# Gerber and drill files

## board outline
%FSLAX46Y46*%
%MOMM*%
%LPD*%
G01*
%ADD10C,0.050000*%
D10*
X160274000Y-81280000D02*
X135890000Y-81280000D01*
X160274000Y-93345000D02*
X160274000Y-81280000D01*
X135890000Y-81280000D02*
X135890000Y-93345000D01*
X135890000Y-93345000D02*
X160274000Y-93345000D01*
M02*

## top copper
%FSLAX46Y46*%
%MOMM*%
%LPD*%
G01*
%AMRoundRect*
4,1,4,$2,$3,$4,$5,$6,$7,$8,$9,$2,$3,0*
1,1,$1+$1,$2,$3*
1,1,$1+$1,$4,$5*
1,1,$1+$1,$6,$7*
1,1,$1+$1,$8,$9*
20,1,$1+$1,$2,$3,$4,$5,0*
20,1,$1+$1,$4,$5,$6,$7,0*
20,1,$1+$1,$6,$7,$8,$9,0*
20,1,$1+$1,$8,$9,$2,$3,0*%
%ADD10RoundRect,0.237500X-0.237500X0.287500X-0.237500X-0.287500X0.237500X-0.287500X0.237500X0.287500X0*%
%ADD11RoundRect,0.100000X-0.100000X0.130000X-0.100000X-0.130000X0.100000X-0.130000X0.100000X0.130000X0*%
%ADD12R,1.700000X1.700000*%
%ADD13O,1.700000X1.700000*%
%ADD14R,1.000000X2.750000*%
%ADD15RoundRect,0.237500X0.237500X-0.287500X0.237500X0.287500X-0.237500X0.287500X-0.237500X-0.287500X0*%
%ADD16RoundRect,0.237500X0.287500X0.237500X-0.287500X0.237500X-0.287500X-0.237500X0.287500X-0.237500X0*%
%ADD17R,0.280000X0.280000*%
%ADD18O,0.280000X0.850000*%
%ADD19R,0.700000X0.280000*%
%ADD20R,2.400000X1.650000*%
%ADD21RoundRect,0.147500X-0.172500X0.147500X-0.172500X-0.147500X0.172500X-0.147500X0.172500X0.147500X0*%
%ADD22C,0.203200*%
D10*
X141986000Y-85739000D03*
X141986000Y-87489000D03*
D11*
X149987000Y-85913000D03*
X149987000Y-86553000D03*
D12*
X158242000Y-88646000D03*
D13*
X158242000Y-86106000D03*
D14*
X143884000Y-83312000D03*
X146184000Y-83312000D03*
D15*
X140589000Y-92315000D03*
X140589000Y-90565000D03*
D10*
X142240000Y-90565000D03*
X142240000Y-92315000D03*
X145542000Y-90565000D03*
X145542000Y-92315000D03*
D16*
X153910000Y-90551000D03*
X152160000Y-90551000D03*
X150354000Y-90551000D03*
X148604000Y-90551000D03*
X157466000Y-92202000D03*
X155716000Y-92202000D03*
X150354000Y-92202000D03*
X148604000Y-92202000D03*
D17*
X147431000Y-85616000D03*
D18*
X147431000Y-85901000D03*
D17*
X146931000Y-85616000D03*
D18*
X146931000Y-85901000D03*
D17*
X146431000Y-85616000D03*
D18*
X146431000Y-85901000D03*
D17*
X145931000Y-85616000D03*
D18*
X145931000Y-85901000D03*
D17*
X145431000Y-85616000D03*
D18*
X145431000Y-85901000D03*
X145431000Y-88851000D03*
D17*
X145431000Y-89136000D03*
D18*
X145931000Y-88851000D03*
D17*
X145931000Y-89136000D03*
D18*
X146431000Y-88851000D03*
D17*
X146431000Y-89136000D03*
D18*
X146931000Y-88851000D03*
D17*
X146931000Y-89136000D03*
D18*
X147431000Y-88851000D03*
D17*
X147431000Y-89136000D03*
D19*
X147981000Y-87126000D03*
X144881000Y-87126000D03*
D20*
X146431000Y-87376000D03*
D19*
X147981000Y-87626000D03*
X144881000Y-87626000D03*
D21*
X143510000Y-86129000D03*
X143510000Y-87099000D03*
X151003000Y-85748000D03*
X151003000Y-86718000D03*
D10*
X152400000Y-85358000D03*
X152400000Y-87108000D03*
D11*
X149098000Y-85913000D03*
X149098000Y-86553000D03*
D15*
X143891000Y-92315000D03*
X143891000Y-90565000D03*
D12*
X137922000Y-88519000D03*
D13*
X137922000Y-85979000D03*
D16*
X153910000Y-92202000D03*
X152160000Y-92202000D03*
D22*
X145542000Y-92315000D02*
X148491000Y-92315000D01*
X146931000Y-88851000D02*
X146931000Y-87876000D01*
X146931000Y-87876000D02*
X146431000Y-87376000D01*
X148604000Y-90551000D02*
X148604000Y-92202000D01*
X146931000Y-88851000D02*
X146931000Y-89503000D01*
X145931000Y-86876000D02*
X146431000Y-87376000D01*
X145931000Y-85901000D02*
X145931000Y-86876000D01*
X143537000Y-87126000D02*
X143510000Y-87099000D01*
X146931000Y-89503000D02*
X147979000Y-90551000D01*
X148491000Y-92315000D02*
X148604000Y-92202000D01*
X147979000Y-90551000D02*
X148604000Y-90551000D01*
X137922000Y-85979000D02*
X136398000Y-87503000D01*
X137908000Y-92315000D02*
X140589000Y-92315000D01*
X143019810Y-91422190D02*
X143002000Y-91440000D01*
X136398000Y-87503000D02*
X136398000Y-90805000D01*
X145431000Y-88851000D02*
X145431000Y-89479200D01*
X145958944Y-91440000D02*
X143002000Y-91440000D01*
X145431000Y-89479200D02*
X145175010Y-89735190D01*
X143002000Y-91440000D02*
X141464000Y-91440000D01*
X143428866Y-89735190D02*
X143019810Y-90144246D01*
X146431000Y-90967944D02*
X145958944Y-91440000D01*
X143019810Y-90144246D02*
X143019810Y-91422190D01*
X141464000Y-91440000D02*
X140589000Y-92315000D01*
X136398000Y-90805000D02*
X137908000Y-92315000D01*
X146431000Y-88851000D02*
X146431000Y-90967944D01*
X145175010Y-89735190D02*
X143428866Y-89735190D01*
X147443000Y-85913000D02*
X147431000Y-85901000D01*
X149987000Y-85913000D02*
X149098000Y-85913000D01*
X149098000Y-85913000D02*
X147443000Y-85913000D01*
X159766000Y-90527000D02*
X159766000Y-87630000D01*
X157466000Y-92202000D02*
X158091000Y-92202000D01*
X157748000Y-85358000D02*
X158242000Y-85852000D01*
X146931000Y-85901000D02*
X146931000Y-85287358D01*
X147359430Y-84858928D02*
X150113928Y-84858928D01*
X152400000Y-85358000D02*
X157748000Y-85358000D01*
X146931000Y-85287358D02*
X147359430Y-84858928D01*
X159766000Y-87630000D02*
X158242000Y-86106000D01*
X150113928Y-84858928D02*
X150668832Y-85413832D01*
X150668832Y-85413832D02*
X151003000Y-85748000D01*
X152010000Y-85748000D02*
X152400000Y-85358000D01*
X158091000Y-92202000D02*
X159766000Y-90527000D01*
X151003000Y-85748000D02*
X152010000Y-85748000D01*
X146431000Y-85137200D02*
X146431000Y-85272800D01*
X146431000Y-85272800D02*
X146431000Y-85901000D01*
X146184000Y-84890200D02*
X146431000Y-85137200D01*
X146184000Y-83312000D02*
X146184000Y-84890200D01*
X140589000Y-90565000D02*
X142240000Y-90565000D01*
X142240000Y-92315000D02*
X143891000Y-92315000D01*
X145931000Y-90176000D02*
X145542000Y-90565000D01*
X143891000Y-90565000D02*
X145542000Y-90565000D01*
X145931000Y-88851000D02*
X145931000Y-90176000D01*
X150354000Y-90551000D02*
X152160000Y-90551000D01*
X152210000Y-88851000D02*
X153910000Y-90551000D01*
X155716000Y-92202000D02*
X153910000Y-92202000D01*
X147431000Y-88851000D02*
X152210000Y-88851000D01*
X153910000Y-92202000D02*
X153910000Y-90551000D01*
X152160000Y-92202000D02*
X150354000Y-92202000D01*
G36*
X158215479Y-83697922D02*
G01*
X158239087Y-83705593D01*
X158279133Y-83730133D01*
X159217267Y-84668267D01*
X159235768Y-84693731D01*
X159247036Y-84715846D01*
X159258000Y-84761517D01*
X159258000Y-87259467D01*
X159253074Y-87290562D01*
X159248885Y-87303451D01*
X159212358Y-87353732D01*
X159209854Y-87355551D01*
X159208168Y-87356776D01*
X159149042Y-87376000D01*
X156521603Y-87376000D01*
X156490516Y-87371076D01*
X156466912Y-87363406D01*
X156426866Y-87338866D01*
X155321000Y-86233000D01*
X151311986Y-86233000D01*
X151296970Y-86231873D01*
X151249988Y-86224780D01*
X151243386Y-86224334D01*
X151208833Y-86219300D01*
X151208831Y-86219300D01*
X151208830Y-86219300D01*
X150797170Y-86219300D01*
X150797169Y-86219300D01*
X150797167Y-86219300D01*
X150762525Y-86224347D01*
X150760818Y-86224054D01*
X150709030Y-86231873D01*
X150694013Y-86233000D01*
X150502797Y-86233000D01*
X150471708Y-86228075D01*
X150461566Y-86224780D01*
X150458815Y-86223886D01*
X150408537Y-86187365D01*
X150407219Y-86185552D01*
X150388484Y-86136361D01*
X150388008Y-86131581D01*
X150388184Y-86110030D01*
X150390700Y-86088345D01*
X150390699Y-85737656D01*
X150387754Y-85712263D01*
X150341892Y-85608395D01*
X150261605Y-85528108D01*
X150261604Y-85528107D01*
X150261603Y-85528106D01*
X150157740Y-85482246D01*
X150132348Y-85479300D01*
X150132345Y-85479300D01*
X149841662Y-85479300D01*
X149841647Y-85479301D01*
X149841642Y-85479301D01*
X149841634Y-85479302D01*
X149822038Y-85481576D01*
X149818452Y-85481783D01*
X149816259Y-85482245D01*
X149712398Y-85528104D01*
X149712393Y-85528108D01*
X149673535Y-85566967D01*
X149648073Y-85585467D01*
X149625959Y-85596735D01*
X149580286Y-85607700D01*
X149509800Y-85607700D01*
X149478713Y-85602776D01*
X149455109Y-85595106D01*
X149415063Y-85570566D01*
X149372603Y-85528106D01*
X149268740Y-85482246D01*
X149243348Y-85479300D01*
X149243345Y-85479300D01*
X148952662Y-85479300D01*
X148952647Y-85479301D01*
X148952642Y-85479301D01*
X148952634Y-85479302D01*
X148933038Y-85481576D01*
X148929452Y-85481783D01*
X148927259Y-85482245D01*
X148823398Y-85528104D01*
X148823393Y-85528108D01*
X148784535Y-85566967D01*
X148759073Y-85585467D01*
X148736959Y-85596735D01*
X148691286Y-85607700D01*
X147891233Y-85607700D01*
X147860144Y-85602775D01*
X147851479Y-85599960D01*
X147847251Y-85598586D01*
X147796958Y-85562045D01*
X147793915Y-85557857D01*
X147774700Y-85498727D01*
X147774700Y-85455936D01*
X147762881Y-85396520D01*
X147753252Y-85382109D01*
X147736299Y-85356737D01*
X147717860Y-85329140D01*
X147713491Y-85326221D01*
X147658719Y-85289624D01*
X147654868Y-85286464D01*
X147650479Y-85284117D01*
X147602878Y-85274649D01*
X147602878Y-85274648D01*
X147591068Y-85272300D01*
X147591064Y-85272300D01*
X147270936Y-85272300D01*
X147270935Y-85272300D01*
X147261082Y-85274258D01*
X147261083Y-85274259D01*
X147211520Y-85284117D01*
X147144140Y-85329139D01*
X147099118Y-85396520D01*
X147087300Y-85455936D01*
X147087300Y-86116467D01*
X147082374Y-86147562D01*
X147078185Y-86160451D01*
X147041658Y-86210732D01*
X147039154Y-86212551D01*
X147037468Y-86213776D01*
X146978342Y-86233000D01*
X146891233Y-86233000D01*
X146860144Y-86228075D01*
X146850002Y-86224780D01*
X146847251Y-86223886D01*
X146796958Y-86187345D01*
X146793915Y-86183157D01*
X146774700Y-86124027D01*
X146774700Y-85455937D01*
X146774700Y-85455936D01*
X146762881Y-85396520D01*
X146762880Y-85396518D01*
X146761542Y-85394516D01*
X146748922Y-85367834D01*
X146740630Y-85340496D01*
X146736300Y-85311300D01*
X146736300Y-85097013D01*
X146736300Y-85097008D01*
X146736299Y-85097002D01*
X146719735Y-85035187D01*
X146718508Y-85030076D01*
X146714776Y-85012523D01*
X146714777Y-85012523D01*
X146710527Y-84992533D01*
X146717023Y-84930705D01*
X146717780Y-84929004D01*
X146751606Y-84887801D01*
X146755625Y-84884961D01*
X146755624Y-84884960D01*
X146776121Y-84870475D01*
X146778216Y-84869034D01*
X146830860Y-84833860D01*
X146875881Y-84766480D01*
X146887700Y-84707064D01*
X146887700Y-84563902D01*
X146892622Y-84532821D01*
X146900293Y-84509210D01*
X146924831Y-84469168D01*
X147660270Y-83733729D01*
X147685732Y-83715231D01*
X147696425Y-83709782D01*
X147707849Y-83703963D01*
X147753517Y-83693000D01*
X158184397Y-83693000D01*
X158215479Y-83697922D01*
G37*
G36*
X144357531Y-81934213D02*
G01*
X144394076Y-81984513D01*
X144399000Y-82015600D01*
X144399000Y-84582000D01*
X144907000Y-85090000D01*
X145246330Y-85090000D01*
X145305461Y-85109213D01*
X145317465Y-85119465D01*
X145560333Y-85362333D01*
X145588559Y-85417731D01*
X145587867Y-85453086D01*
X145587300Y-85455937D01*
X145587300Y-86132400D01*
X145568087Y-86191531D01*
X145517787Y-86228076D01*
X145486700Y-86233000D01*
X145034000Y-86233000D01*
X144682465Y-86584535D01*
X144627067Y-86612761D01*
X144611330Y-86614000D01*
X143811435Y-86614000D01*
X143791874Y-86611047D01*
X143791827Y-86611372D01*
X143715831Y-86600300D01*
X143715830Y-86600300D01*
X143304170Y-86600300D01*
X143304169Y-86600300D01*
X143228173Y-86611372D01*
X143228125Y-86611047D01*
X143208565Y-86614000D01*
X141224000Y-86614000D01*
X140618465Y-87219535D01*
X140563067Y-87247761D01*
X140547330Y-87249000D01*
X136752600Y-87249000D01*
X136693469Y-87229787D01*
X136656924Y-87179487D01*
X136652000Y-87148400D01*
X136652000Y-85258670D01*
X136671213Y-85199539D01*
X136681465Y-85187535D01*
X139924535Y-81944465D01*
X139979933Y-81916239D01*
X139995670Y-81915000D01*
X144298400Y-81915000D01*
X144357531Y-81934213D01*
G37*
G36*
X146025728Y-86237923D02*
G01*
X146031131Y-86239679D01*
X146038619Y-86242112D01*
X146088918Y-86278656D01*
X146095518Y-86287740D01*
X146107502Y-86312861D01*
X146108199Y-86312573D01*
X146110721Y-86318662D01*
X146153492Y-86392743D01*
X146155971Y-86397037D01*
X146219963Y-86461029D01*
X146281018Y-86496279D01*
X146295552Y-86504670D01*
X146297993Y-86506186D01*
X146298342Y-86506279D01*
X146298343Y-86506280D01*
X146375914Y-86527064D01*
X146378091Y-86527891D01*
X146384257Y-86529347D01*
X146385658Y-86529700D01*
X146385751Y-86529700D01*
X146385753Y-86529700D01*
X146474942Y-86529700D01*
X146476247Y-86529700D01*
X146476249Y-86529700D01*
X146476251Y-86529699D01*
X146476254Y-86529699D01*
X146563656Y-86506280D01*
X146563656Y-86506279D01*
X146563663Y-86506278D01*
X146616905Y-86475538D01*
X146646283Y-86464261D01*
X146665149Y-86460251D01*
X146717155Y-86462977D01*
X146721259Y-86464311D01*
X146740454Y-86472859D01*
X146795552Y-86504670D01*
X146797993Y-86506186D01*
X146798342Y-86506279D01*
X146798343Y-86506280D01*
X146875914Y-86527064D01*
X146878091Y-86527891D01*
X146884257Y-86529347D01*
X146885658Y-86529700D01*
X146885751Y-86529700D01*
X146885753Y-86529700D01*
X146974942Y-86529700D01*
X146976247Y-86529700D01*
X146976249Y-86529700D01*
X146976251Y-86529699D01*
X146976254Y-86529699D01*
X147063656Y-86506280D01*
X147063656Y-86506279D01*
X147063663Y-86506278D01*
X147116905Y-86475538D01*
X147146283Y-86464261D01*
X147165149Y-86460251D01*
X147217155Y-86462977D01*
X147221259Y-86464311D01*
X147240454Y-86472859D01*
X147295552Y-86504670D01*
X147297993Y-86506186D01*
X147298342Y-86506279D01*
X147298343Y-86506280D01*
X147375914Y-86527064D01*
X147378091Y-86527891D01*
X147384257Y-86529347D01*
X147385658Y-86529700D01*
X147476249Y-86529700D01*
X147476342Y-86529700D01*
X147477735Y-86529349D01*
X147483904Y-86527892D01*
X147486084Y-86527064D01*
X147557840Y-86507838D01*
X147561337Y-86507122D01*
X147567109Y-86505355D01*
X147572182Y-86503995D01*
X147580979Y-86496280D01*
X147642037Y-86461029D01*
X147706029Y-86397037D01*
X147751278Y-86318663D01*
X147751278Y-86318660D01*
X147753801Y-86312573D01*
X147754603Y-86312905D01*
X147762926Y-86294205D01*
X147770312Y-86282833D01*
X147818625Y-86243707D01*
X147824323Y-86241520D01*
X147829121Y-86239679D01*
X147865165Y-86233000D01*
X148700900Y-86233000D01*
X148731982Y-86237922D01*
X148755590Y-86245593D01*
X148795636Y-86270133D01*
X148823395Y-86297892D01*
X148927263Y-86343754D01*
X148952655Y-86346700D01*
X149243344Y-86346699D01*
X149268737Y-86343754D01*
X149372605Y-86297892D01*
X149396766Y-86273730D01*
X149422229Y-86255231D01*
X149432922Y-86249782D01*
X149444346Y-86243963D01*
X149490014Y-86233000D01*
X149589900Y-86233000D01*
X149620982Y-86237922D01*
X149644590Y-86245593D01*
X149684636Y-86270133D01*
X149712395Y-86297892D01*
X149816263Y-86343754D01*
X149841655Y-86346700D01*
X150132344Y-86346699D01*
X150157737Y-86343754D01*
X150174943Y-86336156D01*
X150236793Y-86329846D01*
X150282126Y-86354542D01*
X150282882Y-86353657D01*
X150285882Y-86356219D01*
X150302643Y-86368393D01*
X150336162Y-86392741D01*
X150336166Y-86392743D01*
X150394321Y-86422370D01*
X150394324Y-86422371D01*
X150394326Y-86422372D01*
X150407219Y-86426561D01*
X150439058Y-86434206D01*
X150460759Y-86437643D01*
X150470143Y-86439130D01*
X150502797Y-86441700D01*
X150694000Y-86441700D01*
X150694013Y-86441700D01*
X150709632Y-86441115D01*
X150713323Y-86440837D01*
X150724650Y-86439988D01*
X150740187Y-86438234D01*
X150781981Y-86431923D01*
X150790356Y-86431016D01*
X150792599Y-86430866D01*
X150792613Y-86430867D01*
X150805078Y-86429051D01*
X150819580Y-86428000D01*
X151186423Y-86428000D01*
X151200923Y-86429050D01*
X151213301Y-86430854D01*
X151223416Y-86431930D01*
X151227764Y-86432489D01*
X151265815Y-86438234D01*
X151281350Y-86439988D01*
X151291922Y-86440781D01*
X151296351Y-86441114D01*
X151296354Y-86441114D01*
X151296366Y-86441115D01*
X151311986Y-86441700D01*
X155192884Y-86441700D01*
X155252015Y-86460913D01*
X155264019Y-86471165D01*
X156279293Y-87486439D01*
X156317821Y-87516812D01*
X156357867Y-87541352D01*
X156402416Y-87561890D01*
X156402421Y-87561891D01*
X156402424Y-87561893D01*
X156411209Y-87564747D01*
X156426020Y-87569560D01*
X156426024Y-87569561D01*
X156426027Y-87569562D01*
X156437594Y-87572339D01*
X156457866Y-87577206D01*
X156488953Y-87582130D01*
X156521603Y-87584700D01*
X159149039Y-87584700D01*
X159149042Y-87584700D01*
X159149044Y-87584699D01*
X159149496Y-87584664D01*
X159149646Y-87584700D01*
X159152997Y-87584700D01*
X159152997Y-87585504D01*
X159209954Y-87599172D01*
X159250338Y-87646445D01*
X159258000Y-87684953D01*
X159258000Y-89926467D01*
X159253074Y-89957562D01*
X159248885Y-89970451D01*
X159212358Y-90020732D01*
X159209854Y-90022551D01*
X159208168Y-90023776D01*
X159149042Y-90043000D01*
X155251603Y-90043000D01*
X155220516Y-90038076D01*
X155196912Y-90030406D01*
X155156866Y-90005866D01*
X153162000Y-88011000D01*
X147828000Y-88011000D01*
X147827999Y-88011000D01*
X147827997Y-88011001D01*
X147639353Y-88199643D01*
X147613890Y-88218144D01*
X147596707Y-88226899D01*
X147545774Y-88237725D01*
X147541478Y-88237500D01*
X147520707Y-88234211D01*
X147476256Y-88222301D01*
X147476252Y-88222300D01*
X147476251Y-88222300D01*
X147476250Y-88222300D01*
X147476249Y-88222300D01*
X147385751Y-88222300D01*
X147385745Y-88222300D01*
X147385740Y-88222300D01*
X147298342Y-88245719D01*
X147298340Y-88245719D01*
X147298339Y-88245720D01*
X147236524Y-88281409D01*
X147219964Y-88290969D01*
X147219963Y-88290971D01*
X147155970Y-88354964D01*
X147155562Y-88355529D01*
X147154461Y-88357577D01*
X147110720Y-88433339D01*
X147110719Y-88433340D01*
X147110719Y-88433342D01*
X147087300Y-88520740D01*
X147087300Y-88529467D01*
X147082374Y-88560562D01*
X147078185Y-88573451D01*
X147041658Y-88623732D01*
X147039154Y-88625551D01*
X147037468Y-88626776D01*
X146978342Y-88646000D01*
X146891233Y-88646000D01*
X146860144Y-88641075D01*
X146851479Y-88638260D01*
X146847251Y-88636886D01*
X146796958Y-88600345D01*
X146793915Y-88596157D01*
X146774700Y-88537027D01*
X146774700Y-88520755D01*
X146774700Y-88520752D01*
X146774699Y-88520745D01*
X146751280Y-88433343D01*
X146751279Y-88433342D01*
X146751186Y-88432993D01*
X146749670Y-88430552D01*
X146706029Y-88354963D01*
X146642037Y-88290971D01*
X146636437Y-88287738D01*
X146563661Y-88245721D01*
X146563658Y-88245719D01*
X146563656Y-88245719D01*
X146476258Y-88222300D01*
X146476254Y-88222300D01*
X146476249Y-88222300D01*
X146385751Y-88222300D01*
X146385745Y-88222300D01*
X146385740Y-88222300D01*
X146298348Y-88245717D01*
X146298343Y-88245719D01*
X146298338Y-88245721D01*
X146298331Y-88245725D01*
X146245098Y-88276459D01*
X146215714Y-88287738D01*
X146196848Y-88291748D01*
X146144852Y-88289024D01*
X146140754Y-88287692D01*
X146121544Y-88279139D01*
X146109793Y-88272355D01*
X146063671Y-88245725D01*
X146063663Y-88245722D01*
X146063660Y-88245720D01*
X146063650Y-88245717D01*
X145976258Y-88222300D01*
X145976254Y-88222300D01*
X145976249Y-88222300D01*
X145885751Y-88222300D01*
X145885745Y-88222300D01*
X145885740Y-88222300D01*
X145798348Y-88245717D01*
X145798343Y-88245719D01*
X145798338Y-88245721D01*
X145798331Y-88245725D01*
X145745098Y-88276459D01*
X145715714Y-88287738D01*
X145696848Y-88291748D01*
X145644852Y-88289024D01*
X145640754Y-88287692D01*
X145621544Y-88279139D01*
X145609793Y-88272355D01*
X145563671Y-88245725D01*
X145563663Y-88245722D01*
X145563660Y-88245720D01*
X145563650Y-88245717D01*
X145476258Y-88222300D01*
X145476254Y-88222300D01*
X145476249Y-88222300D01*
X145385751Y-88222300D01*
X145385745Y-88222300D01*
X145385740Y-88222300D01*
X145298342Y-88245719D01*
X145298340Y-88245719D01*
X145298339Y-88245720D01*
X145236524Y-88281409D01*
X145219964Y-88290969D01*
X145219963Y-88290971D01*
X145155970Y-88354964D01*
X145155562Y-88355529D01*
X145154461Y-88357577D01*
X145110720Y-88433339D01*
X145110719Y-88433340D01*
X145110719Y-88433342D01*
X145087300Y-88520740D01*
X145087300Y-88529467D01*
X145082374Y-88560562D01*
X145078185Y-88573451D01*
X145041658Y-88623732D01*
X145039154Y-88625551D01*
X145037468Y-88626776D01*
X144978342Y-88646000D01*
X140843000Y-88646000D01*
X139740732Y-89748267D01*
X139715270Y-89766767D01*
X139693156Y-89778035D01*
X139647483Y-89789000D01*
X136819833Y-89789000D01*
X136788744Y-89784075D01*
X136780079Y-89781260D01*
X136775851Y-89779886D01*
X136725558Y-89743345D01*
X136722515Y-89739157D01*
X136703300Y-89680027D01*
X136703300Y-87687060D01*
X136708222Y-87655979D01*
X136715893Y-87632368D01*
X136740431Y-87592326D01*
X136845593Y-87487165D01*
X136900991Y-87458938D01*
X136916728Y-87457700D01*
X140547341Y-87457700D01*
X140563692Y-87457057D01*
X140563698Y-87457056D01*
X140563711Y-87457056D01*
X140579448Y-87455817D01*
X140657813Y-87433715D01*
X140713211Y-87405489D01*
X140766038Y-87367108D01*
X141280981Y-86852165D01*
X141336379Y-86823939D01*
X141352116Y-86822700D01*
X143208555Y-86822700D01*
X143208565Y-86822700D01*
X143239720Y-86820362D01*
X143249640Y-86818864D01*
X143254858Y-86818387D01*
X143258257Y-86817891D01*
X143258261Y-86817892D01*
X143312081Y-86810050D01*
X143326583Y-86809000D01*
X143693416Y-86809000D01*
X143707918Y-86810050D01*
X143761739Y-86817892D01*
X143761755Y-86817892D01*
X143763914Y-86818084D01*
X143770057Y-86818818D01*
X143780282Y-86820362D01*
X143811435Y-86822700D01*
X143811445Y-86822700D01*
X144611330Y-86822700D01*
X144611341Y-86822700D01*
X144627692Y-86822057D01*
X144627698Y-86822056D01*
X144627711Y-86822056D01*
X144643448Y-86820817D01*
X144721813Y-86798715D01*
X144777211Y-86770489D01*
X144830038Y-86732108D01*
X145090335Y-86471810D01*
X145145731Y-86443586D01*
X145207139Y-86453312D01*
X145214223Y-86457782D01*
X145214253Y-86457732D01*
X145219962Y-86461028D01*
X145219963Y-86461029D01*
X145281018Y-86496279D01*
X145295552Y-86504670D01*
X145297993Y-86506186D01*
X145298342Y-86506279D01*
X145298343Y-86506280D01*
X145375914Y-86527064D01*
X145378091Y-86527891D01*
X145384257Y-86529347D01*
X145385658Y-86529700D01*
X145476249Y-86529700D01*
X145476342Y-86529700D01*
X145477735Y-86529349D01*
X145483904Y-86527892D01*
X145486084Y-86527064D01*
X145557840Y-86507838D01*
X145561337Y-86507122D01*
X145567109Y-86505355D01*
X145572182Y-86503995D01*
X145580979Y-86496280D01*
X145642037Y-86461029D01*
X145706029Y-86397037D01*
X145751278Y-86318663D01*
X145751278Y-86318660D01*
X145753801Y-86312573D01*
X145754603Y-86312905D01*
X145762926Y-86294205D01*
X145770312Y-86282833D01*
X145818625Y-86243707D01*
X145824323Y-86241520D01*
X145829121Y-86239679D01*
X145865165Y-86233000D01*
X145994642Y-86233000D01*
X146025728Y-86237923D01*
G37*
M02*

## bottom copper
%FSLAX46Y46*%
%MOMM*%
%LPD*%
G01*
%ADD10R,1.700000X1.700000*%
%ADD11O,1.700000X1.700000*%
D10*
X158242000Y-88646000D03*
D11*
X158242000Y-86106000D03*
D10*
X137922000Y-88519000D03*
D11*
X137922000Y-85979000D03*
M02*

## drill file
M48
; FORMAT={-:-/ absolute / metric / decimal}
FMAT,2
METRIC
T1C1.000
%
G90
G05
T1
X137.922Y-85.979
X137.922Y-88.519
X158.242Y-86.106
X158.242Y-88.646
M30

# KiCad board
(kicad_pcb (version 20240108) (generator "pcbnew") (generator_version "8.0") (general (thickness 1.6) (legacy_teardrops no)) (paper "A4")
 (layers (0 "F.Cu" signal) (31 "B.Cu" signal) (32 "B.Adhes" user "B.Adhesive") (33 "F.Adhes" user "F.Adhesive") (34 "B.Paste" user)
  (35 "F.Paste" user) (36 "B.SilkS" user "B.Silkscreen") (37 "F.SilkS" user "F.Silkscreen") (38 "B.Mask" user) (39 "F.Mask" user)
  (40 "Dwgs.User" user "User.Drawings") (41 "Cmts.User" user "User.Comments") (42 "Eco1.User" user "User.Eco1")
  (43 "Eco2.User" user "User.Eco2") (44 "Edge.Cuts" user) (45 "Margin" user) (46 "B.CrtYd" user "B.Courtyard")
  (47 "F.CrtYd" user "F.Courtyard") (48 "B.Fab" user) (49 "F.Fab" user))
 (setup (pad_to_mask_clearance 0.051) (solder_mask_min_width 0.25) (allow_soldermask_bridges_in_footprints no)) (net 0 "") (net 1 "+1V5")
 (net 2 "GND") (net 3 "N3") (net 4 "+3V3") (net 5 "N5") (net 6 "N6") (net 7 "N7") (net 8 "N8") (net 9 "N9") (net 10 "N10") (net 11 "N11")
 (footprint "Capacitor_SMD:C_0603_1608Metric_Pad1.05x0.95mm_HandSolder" (layer "F.Cu") (at 141.986 86.614 -90)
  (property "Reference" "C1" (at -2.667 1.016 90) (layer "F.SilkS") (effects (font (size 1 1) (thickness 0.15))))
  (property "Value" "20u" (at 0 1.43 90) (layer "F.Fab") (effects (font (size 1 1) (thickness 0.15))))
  (pad "1" smd roundrect (at -0.875 0 270) (size 1.05 0.95) (layers "F.Cu" "F.Paste" "F.Mask") (roundrect_rratio 0.25) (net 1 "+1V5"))
  (pad "2" smd roundrect (at 0.875 0 270) (size 1.05 0.95) (layers "F.Cu" "F.Paste" "F.Mask") (roundrect_rratio 0.25) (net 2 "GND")))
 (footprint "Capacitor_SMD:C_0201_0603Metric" (layer "F.Cu") (at 149.987 86.233 -90)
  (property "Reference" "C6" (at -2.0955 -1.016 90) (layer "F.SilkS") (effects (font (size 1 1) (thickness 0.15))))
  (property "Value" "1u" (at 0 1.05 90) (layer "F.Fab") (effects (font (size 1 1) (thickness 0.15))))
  (pad "" smd roundrect (at -0.345 0 270) (size 0.318 0.36) (layers "F.Paste") (roundrect_rratio 0.25))
  (pad "" smd roundrect (at 0.345 0 270) (size 0.318 0.36) (layers "F.Paste") (roundrect_rratio 0.25))
  (pad "1" smd roundrect (at -0.32 0 270) (size 0.46 0.4) (layers "F.Cu" "F.Mask") (roundrect_rratio 0.25) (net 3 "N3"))
  (pad "2" smd roundrect (at 0.32 0 270) (size 0.46 0.4) (layers "F.Cu" "F.Mask") (roundrect_rratio 0.25) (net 2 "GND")))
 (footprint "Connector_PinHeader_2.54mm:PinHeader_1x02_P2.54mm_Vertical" (layer "F.Cu") (at 158.242 88.646 180)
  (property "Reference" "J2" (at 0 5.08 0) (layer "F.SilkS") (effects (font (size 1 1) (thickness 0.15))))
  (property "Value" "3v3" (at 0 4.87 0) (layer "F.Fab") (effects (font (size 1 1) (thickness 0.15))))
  (pad "1" thru_hole rect (at 0 0 180) (size 1.7 1.7) (drill 1) (layers "*.Cu" "*.Mask") (remove_unused_layers no) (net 2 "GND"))
  (pad "2" thru_hole oval (at 0 2.54 180) (size 1.7 1.7) (drill 1) (layers "*.Cu" "*.Mask") (remove_unused_layers no) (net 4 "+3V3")))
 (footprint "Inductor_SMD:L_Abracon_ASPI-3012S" (layer "F.Cu") (at 145.034 83.312)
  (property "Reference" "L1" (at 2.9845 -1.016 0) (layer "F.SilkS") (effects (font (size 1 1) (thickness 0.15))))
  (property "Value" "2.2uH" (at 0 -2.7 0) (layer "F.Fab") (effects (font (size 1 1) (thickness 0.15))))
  (pad "1" smd rect (at -1.15 0) (size 1 2.75) (layers "F.Cu" "F.Paste" "F.Mask") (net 1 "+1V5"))
  (pad "2" smd rect (at 1.15 0) (size 1 2.75) (layers "F.Cu" "F.Paste" "F.Mask") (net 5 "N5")))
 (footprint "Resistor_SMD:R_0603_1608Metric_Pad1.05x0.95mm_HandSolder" (layer "F.Cu") (at 140.589 91.44 90)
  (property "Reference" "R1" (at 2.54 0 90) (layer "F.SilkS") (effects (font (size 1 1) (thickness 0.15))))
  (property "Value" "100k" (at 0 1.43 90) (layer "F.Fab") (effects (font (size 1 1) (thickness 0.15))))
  (pad "1" smd roundrect (at -0.875 0 90) (size 1.05 0.95) (layers "F.Cu" "F.Paste" "F.Mask") (roundrect_rratio 0.25) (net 1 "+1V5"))
  (pad "2" smd roundrect (at 0.875 0 90) (size 1.05 0.95) (layers "F.Cu" "F.Paste" "F.Mask") (roundrect_rratio 0.25) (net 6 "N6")))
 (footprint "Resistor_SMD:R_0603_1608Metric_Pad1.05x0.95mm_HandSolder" (layer "F.Cu") (at 142.24 91.44 -90)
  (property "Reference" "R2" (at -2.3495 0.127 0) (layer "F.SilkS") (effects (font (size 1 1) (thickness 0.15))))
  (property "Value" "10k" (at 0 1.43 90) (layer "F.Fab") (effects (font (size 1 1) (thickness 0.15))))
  (pad "1" smd roundrect (at -0.875 0 270) (size 1.05 0.95) (layers "F.Cu" "F.Paste" "F.Mask") (roundrect_rratio 0.25) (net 6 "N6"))
  (pad "2" smd roundrect (at 0.875 0 270) (size 1.05 0.95) (layers "F.Cu" "F.Paste" "F.Mask") (roundrect_rratio 0.25) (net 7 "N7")))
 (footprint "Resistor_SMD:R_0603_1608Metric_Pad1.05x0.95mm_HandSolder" (layer "F.Cu") (at 145.542 91.44 -90)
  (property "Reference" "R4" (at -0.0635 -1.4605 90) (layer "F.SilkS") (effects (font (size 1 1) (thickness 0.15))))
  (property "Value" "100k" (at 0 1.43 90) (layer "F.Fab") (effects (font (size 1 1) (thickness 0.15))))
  (pad "1" smd roundrect (at -0.875 0 270) (size 1.05 0.95) (layers "F.Cu" "F.Paste" "F.Mask") (roundrect_rratio 0.25) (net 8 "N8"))
  (pad "2" smd roundrect (at 0.875 0 270) (size 1.05 0.95) (layers "F.Cu" "F.Paste" "F.Mask") (roundrect_rratio 0.25) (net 2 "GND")))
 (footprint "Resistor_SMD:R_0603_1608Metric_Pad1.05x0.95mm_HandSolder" (layer "F.Cu") (at 153.035 90.551 180)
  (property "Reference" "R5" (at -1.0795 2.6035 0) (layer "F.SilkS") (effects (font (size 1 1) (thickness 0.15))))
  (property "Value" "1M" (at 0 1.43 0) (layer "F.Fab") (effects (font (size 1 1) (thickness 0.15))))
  (pad "1" smd roundrect (at -0.875 0 180) (size 1.05 0.95) (layers "F.Cu" "F.Paste" "F.Mask") (roundrect_rratio 0.25) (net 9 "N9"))
  (pad "2" smd roundrect (at 0.875 0 180) (size 1.05 0.95) (layers "F.Cu" "F.Paste" "F.Mask") (roundrect_rratio 0.25) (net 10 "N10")))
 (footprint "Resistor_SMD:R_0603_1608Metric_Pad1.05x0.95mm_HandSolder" (layer "F.Cu") (at 149.479 90.551 180)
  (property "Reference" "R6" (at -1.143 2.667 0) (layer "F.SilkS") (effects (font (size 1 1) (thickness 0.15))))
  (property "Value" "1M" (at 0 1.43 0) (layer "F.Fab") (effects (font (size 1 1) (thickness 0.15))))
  (pad "1" smd roundrect (at -0.875 0 180) (size 1.05 0.95) (layers "F.Cu" "F.Paste" "F.Mask") (roundrect_rratio 0.25) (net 10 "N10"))
  (pad "2" smd roundrect (at 0.875 0 180) (size 1.05 0.95) (layers "F.Cu" "F.Paste" "F.Mask") (roundrect_rratio 0.25) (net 2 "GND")))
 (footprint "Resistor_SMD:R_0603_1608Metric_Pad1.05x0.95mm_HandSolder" (layer "F.Cu") (at 156.591 92.202 180)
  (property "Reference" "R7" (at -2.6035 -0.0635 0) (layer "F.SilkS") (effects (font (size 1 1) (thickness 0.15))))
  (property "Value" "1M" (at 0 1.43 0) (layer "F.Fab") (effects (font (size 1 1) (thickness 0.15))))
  (pad "1" smd roundrect (at -0.875 0 180) (size 1.05 0.95) (layers "F.Cu" "F.Paste" "F.Mask") (roundrect_rratio 0.25) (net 4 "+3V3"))
  (pad "2" smd roundrect (at 0.875 0 180) (size 1.05 0.95) (layers "F.Cu" "F.Paste" "F.Mask") (roundrect_rratio 0.25) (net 9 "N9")))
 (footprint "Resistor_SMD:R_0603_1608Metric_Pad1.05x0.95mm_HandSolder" (layer "F.Cu") (at 149.479 92.202 180)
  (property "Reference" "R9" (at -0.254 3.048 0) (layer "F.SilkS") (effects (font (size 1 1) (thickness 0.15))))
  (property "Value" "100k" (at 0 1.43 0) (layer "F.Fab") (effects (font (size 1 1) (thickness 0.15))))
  (pad "1" smd roundrect (at -0.875 0 180) (size 1.05 0.95) (layers "F.Cu" "F.Paste" "F.Mask") (roundrect_rratio 0.25) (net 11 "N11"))
  (pad "2" smd roundrect (at 0.875 0 180) (size 1.05 0.95) (layers "F.Cu" "F.Paste" "F.Mask") (roundrect_rratio 0.25) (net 2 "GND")))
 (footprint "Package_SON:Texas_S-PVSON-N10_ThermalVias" (layer "F.Cu") (at 146.431 87.376 -90)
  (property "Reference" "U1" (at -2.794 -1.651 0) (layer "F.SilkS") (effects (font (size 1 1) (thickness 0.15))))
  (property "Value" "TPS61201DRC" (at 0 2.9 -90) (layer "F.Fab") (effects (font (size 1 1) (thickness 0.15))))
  (pad "1" smd rect (at -1.76 -1 270) (size 0.28 0.28) (layers "F.Cu" "F.Paste" "F.Mask") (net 3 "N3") (solder_mask_margin 0.07)
   (solder_paste_margin -0.025))
  (pad "1" smd oval (at -1.475 -1 270) (size 0.85 0.28) (layers "F.Cu" "F.Paste" "F.Mask") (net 3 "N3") (solder_mask_margin 0.07)
   (solder_paste_margin -0.025))
  (pad "2" smd rect (at -1.76 -0.5 270) (size 0.28 0.28) (layers "F.Cu" "F.Paste" "F.Mask") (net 4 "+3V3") (solder_mask_margin 0.07)
   (solder_paste_margin -0.025))
  (pad "2" smd oval (at -1.475 -0.5 270) (size 0.85 0.28) (layers "F.Cu" "F.Paste" "F.Mask") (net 4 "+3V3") (solder_mask_margin 0.07)
   (solder_paste_margin -0.025))
  (pad "3" smd rect (at -1.76 0 270) (size 0.28 0.28) (layers "F.Cu" "F.Paste" "F.Mask") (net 5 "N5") (solder_mask_margin 0.07)
   (solder_paste_margin -0.025))
  (pad "3" smd oval (at -1.475 0 270) (size 0.85 0.28) (layers "F.Cu" "F.Paste" "F.Mask") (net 5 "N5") (solder_mask_margin 0.07)
   (solder_paste_margin -0.025))
  (pad "4" smd rect (at -1.76 0.5 270) (size 0.28 0.28) (layers "F.Cu" "F.Paste" "F.Mask") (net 2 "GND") (solder_mask_margin 0.07)
   (solder_paste_margin -0.025))
  (pad "4" smd oval (at -1.475 0.5 270) (size 0.85 0.28) (layers "F.Cu" "F.Paste" "F.Mask") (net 2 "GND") (solder_mask_margin 0.07)
   (solder_paste_margin -0.025))
  (pad "5" smd rect (at -1.76 1 270) (size 0.28 0.28) (layers "F.Cu" "F.Paste" "F.Mask") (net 1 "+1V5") (solder_mask_margin 0.07)
   (solder_paste_margin -0.025))
  (pad "5" smd oval (at -1.475 1 270) (size 0.85 0.28) (layers "F.Cu" "F.Paste" "F.Mask") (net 1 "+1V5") (solder_mask_margin 0.07)
   (solder_paste_margin -0.025))
  (pad "6" smd oval (at 1.475 1 270) (size 0.85 0.28) (layers "F.Cu" "F.Paste" "F.Mask") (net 1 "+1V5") (solder_mask_margin 0.07)
   (solder_paste_margin -0.025))
  (pad "6" smd rect (at 1.76 1 270) (size 0.28 0.28) (layers "F.Cu" "F.Paste" "F.Mask") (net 1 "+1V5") (solder_mask_margin 0.07)
   (solder_paste_margin -0.025))
  (pad "7" smd oval (at 1.475 0.5 270) (size 0.85 0.28) (layers "F.Cu" "F.Paste" "F.Mask") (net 8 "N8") (solder_mask_margin 0.07)
   (solder_paste_margin -0.025))
  (pad "7" smd rect (at 1.76 0.5 270) (size 0.28 0.28) (layers "F.Cu" "F.Paste" "F.Mask") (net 8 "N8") (solder_mask_margin 0.07)
   (solder_paste_margin -0.025))
  (pad "8" smd oval (at 1.475 0 270) (size 0.85 0.28) (layers "F.Cu" "F.Paste" "F.Mask") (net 1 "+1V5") (solder_mask_margin 0.07)
   (solder_paste_margin -0.025))
  (pad "8" smd rect (at 1.76 0 270) (size 0.28 0.28) (layers "F.Cu" "F.Paste" "F.Mask") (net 1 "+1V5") (solder_mask_margin 0.07)
   (solder_paste_margin -0.025))
  (pad "9" smd oval (at 1.475 -0.5 270) (size 0.85 0.28) (layers "F.Cu" "F.Paste" "F.Mask") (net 2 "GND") (solder_mask_margin 0.07)
   (solder_paste_margin -0.025))
  (pad "9" smd rect (at 1.76 -0.5 270) (size 0.28 0.28) (layers "F.Cu" "F.Paste" "F.Mask") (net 2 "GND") (solder_mask_margin 0.07)
   (solder_paste_margin -0.025))
  (pad "10" smd oval (at 1.475 -1 270) (size 0.85 0.28) (layers "F.Cu" "F.Paste" "F.Mask") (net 9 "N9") (solder_mask_margin 0.07)
   (solder_paste_margin -0.025))
  (pad "10" smd rect (at 1.76 -1 270) (size 0.28 0.28) (layers "F.Cu" "F.Paste" "F.Mask") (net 9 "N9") (solder_mask_margin 0.07)
   (solder_paste_margin -0.025))
  (pad "11" smd rect (at -0.25 -1.55 270) (size 0.28 0.7) (layers "F.Cu" "F.Mask") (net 2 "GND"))
  (pad "11" smd rect (at -0.25 1.55 270) (size 0.28 0.7) (layers "F.Cu" "F.Mask") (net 2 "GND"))
  (pad "11" smd rect (at 0 0 270) (size 1.65 2.4) (layers "F.Cu" "F.Mask") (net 2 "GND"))
  (pad "11" smd rect (at 0.25 -1.55 270) (size 0.28 0.7) (layers "F.Cu" "F.Mask") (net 2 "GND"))
  (pad "11" smd rect (at 0.25 1.55 270) (size 0.28 0.7) (layers "F.Cu" "F.Mask") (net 2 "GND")))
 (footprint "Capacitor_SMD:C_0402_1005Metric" (layer "F.Cu") (at 143.51 86.614 -90)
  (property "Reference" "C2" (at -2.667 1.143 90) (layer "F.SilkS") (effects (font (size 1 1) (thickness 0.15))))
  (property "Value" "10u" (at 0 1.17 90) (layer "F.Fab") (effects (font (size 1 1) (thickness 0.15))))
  (pad "1" smd roundrect (at -0.485 0 270) (size 0.59 0.64) (layers "F.Cu" "F.Paste" "F.Mask") (roundrect_rratio 0.25) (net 1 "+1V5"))
  (pad "2" smd roundrect (at 0.485 0 270) (size 0.59 0.64) (layers "F.Cu" "F.Paste" "F.Mask") (roundrect_rratio 0.25) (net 2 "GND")))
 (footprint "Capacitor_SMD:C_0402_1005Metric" (layer "F.Cu") (at 151.003 86.233 -90)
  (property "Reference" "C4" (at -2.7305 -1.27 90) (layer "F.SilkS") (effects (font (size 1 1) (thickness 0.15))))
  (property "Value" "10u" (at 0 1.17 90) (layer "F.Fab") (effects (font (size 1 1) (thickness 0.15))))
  (pad "1" smd roundrect (at -0.485 0 270) (size 0.59 0.64) (layers "F.Cu" "F.Paste" "F.Mask") (roundrect_rratio 0.25) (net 4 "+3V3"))
  (pad "2" smd roundrect (at 0.485 0 270) (size 0.59 0.64) (layers "F.Cu" "F.Paste" "F.Mask") (roundrect_rratio 0.25) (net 2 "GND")))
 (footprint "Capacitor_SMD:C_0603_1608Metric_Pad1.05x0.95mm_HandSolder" (layer "F.Cu") (at 152.4 86.233 -90)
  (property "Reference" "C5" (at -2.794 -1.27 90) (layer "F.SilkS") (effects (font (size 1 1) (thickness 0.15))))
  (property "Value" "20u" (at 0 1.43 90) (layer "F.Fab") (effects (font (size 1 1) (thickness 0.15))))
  (pad "1" smd roundrect (at -0.875 0 270) (size 1.05 0.95) (layers "F.Cu" "F.Paste" "F.Mask") (roundrect_rratio 0.25) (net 4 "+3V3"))
  (pad "2" smd roundrect (at 0.875 0 270) (size 1.05 0.95) (layers "F.Cu" "F.Paste" "F.Mask") (roundrect_rratio 0.25) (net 2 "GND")))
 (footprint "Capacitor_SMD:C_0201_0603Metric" (layer "F.Cu") (at 149.098 86.233 -90)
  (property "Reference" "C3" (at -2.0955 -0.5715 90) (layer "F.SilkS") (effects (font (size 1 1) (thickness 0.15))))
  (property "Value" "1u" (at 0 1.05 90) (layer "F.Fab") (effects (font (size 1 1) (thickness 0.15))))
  (pad "" smd roundrect (at -0.345 0 270) (size 0.318 0.36) (layers "F.Paste") (roundrect_rratio 0.25))
  (pad "" smd roundrect (at 0.345 0 270) (size 0.318 0.36) (layers "F.Paste") (roundrect_rratio 0.25))
  (pad "1" smd roundrect (at -0.32 0 270) (size 0.46 0.4) (layers "F.Cu" "F.Mask") (roundrect_rratio 0.25) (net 3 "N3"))
  (pad "2" smd roundrect (at 0.32 0 270) (size 0.46 0.4) (layers "F.Cu" "F.Mask") (roundrect_rratio 0.25) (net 2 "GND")))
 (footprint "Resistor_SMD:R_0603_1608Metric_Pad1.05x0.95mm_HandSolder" (layer "F.Cu") (at 143.891 91.44 90)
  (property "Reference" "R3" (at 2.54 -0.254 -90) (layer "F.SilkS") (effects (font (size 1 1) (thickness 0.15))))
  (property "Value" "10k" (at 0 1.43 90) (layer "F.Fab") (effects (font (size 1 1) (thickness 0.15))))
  (pad "1" smd roundrect (at -0.875 0 90) (size 1.05 0.95) (layers "F.Cu" "F.Paste" "F.Mask") (roundrect_rratio 0.25) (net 7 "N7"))
  (pad "2" smd roundrect (at 0.875 0 90) (size 1.05 0.95) (layers "F.Cu" "F.Paste" "F.Mask") (roundrect_rratio 0.25) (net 8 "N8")))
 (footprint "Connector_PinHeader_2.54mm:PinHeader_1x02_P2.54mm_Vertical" (layer "F.Cu") (at 137.922 88.519 180)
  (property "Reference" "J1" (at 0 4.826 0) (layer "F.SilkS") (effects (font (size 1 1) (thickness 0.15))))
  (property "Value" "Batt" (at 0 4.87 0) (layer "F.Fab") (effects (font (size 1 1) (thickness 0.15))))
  (pad "1" thru_hole rect (at 0 0 180) (size 1.7 1.7) (drill 1) (layers "*.Cu" "*.Mask") (remove_unused_layers no) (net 2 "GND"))
  (pad "2" thru_hole oval (at 0 2.54 180) (size 1.7 1.7) (drill 1) (layers "*.Cu" "*.Mask") (remove_unused_layers no) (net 1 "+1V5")))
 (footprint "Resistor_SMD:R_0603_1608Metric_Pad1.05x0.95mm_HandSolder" (layer "F.Cu") (at 153.035 92.202 180)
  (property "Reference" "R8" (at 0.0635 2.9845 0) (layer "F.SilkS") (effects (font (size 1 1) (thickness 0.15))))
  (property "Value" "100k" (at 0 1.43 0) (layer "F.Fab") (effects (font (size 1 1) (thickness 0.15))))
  (pad "1" smd roundrect (at -0.875 0 180) (size 1.05 0.95) (layers "F.Cu" "F.Paste" "F.Mask") (roundrect_rratio 0.25) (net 9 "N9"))
  (pad "2" smd roundrect (at 0.875 0 180) (size 1.05 0.95) (layers "F.Cu" "F.Paste" "F.Mask") (roundrect_rratio 0.25) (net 11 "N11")))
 (gr_line (start 160.274 81.28) (end 135.89 81.28) (stroke (width 0.05) (type solid)) (layer "Edge.Cuts"))
 (gr_line (start 160.274 93.345) (end 160.274 81.28) (stroke (width 0.05) (type solid)) (layer "Edge.Cuts"))
 (gr_line (start 135.89 81.28) (end 135.89 93.345) (stroke (width 0.05) (type solid)) (layer "Edge.Cuts"))
 (gr_line (start 135.89 93.345) (end 160.274 93.345) (stroke (width 0.05) (type solid)) (layer "Edge.Cuts"))
 (segment (start 145.542 92.315) (end 148.491 92.315) (width 0.2032) (layer "F.Cu") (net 2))
 (segment (start 146.931 88.851) (end 146.931 87.876) (width 0.2032) (layer "F.Cu") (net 2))
 (segment (start 146.931 87.876) (end 146.431 87.376) (width 0.2032) (layer "F.Cu") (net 2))
 (segment (start 148.604 90.551) (end 148.604 92.202) (width 0.2032) (layer "F.Cu") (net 2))
 (segment (start 146.931 88.851) (end 146.931 89.503) (width 0.2032) (layer "F.Cu") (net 2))
 (segment (start 145.931 86.876) (end 146.431 87.376) (width 0.2032) (layer "F.Cu") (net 2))
 (segment (start 145.931 85.901) (end 145.931 86.876) (width 0.2032) (layer "F.Cu") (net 2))
 (segment (start 143.537 87.126) (end 143.51 87.099) (width 0.2032) (layer "F.Cu") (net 2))
 (segment (start 146.931 89.503) (end 147.979 90.551) (width 0.2032) (layer "F.Cu") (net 2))
 (segment (start 148.491 92.315) (end 148.604 92.202) (width 0.2032) (layer "F.Cu") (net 2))
 (segment (start 147.979 90.551) (end 148.604 90.551) (width 0.2032) (layer "F.Cu") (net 2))
 (segment (start 137.922 85.979) (end 136.398 87.503) (width 0.2032) (layer "F.Cu") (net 1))
 (segment (start 137.908 92.315) (end 140.589 92.315) (width 0.2032) (layer "F.Cu") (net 1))
 (segment (start 143.01981 91.42219) (end 143.002 91.44) (width 0.2032) (layer "F.Cu") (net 1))
 (segment (start 136.398 87.503) (end 136.398 90.805) (width 0.2032) (layer "F.Cu") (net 1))
 (segment (start 145.431 88.851) (end 145.431 89.4792) (width 0.2032) (layer "F.Cu") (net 1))
 (segment (start 145.958944 91.44) (end 143.002 91.44) (width 0.2032) (layer "F.Cu") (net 1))
 (segment (start 145.431 89.4792) (end 145.17501 89.73519) (width 0.2032) (layer "F.Cu") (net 1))
 (segment (start 143.002 91.44) (end 141.464 91.44) (width 0.2032) (layer "F.Cu") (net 1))
 (segment (start 143.428866 89.73519) (end 143.01981 90.144246) (width 0.2032) (layer "F.Cu") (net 1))
 (segment (start 146.431 90.967944) (end 145.958944 91.44) (width 0.2032) (layer "F.Cu") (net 1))
 (segment (start 143.01981 90.144246) (end 143.01981 91.42219) (width 0.2032) (layer "F.Cu") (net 1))
 (segment (start 141.464 91.44) (end 140.589 92.315) (width 0.2032) (layer "F.Cu") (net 1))
 (segment (start 136.398 90.805) (end 137.908 92.315) (width 0.2032) (layer "F.Cu") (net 1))
 (segment (start 146.431 88.851) (end 146.431 90.967944) (width 0.2032) (layer "F.Cu") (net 1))
 (segment (start 145.17501 89.73519) (end 143.428866 89.73519) (width 0.2032) (layer "F.Cu") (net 1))
 (segment (start 147.443 85.913) (end 147.431 85.901) (width 0.2032) (layer "F.Cu") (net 3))
 (segment (start 149.987 85.913) (end 149.098 85.913) (width 0.2032) (layer "F.Cu") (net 3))
 (segment (start 149.098 85.913) (end 147.443 85.913) (width 0.2032) (layer "F.Cu") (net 3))
 (segment (start 159.766 90.527) (end 159.766 87.63) (width 0.2032) (layer "F.Cu") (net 4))
 (segment (start 157.466 92.202) (end 158.091 92.202) (width 0.2032) (layer "F.Cu") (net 4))
 (segment (start 157.748 85.358) (end 158.242 85.852) (width 0.2032) (layer "F.Cu") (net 4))
 (segment (start 146.931 85.901) (end 146.931 85.287358) (width 0.2032) (layer "F.Cu") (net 4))
 (segment (start 147.35943 84.858928) (end 150.113928 84.858928) (width 0.2032) (layer "F.Cu") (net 4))
 (segment (start 152.4 85.358) (end 157.748 85.358) (width 0.2032) (layer "F.Cu") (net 4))
 (segment (start 146.931 85.287358) (end 147.35943 84.858928) (width 0.2032) (layer "F.Cu") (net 4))
 (segment (start 159.766 87.63) (end 158.242 86.106) (width 0.2032) (layer "F.Cu") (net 4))
 (segment (start 150.113928 84.858928) (end 150.668832 85.413832) (width 0.2032) (layer "F.Cu") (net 4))
 (segment (start 150.668832 85.413832) (end 151.003 85.748) (width 0.2032) (layer "F.Cu") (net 4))
 (segment (start 152.01 85.748) (end 152.4 85.358) (width 0.2032) (layer "F.Cu") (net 4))
 (segment (start 158.091 92.202) (end 159.766 90.527) (width 0.2032) (layer "F.Cu") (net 4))
 (segment (start 151.003 85.748) (end 152.01 85.748) (width 0.2032) (layer "F.Cu") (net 4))
 (segment (start 146.431 85.1372) (end 146.431 85.2728) (width 0.2032) (layer "F.Cu") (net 5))
 (segment (start 146.431 85.2728) (end 146.431 85.901) (width 0.2032) (layer "F.Cu") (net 5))
 (segment (start 146.184 84.8902) (end 146.431 85.1372) (width 0.2032) (layer "F.Cu") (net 5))
 (segment (start 146.184 83.312) (end 146.184 84.8902) (width 0.2032) (layer "F.Cu") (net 5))
 (segment (start 140.589 90.565) (end 142.24 90.565) (width 0.2032) (layer "F.Cu") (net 6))
 (segment (start 142.24 92.315) (end 143.891 92.315) (width 0.2032) (layer "F.Cu") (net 7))
 (segment (start 145.931 90.176) (end 145.542 90.565) (width 0.2032) (layer "F.Cu") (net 8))
 (segment (start 143.891 90.565) (end 145.542 90.565) (width 0.2032) (layer "F.Cu") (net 8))
 (segment (start 145.931 88.851) (end 145.931 90.176) (width 0.2032) (layer "F.Cu") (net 8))
 (segment (start 150.354 90.551) (end 152.16 90.551) (width 0.2032) (layer "F.Cu") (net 10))
 (segment (start 152.21 88.851) (end 153.91 90.551) (width 0.2032) (layer "F.Cu") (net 9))
 (segment (start 155.716 92.202) (end 153.91 92.202) (width 0.2032) (layer "F.Cu") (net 9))
 (segment (start 147.431 88.851) (end 152.21 88.851) (width 0.2032) (layer "F.Cu") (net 9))
 (segment (start 153.91 92.202) (end 153.91 90.551) (width 0.2032) (layer "F.Cu") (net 9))
 (segment (start 152.16 92.202) (end 150.354 92.202) (width 0.2032) (layer "F.Cu") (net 11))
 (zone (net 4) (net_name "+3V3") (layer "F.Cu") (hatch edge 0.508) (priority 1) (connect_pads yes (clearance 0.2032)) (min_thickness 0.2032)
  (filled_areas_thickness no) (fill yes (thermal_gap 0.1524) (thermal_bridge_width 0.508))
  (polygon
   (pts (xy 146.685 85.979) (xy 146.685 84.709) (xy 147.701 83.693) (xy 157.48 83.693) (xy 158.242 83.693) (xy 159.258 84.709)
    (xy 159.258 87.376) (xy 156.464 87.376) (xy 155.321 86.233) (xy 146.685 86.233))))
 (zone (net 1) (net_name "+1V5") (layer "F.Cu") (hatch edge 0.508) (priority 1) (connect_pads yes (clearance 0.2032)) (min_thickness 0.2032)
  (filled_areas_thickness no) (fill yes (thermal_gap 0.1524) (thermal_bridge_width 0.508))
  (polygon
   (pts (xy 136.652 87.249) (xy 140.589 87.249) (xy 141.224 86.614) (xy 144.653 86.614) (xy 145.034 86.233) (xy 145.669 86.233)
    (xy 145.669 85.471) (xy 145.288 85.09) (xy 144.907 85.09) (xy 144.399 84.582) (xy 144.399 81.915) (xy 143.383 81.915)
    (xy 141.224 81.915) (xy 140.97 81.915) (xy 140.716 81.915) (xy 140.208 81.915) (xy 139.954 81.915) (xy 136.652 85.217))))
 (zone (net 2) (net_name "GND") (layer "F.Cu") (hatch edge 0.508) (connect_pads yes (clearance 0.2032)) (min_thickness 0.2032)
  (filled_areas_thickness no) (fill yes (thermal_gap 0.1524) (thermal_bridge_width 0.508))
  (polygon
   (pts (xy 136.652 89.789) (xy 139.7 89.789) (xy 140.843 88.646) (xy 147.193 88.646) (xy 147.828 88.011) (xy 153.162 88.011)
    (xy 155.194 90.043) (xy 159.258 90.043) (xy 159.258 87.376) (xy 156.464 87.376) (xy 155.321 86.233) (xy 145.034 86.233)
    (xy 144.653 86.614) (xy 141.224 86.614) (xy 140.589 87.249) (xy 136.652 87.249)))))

